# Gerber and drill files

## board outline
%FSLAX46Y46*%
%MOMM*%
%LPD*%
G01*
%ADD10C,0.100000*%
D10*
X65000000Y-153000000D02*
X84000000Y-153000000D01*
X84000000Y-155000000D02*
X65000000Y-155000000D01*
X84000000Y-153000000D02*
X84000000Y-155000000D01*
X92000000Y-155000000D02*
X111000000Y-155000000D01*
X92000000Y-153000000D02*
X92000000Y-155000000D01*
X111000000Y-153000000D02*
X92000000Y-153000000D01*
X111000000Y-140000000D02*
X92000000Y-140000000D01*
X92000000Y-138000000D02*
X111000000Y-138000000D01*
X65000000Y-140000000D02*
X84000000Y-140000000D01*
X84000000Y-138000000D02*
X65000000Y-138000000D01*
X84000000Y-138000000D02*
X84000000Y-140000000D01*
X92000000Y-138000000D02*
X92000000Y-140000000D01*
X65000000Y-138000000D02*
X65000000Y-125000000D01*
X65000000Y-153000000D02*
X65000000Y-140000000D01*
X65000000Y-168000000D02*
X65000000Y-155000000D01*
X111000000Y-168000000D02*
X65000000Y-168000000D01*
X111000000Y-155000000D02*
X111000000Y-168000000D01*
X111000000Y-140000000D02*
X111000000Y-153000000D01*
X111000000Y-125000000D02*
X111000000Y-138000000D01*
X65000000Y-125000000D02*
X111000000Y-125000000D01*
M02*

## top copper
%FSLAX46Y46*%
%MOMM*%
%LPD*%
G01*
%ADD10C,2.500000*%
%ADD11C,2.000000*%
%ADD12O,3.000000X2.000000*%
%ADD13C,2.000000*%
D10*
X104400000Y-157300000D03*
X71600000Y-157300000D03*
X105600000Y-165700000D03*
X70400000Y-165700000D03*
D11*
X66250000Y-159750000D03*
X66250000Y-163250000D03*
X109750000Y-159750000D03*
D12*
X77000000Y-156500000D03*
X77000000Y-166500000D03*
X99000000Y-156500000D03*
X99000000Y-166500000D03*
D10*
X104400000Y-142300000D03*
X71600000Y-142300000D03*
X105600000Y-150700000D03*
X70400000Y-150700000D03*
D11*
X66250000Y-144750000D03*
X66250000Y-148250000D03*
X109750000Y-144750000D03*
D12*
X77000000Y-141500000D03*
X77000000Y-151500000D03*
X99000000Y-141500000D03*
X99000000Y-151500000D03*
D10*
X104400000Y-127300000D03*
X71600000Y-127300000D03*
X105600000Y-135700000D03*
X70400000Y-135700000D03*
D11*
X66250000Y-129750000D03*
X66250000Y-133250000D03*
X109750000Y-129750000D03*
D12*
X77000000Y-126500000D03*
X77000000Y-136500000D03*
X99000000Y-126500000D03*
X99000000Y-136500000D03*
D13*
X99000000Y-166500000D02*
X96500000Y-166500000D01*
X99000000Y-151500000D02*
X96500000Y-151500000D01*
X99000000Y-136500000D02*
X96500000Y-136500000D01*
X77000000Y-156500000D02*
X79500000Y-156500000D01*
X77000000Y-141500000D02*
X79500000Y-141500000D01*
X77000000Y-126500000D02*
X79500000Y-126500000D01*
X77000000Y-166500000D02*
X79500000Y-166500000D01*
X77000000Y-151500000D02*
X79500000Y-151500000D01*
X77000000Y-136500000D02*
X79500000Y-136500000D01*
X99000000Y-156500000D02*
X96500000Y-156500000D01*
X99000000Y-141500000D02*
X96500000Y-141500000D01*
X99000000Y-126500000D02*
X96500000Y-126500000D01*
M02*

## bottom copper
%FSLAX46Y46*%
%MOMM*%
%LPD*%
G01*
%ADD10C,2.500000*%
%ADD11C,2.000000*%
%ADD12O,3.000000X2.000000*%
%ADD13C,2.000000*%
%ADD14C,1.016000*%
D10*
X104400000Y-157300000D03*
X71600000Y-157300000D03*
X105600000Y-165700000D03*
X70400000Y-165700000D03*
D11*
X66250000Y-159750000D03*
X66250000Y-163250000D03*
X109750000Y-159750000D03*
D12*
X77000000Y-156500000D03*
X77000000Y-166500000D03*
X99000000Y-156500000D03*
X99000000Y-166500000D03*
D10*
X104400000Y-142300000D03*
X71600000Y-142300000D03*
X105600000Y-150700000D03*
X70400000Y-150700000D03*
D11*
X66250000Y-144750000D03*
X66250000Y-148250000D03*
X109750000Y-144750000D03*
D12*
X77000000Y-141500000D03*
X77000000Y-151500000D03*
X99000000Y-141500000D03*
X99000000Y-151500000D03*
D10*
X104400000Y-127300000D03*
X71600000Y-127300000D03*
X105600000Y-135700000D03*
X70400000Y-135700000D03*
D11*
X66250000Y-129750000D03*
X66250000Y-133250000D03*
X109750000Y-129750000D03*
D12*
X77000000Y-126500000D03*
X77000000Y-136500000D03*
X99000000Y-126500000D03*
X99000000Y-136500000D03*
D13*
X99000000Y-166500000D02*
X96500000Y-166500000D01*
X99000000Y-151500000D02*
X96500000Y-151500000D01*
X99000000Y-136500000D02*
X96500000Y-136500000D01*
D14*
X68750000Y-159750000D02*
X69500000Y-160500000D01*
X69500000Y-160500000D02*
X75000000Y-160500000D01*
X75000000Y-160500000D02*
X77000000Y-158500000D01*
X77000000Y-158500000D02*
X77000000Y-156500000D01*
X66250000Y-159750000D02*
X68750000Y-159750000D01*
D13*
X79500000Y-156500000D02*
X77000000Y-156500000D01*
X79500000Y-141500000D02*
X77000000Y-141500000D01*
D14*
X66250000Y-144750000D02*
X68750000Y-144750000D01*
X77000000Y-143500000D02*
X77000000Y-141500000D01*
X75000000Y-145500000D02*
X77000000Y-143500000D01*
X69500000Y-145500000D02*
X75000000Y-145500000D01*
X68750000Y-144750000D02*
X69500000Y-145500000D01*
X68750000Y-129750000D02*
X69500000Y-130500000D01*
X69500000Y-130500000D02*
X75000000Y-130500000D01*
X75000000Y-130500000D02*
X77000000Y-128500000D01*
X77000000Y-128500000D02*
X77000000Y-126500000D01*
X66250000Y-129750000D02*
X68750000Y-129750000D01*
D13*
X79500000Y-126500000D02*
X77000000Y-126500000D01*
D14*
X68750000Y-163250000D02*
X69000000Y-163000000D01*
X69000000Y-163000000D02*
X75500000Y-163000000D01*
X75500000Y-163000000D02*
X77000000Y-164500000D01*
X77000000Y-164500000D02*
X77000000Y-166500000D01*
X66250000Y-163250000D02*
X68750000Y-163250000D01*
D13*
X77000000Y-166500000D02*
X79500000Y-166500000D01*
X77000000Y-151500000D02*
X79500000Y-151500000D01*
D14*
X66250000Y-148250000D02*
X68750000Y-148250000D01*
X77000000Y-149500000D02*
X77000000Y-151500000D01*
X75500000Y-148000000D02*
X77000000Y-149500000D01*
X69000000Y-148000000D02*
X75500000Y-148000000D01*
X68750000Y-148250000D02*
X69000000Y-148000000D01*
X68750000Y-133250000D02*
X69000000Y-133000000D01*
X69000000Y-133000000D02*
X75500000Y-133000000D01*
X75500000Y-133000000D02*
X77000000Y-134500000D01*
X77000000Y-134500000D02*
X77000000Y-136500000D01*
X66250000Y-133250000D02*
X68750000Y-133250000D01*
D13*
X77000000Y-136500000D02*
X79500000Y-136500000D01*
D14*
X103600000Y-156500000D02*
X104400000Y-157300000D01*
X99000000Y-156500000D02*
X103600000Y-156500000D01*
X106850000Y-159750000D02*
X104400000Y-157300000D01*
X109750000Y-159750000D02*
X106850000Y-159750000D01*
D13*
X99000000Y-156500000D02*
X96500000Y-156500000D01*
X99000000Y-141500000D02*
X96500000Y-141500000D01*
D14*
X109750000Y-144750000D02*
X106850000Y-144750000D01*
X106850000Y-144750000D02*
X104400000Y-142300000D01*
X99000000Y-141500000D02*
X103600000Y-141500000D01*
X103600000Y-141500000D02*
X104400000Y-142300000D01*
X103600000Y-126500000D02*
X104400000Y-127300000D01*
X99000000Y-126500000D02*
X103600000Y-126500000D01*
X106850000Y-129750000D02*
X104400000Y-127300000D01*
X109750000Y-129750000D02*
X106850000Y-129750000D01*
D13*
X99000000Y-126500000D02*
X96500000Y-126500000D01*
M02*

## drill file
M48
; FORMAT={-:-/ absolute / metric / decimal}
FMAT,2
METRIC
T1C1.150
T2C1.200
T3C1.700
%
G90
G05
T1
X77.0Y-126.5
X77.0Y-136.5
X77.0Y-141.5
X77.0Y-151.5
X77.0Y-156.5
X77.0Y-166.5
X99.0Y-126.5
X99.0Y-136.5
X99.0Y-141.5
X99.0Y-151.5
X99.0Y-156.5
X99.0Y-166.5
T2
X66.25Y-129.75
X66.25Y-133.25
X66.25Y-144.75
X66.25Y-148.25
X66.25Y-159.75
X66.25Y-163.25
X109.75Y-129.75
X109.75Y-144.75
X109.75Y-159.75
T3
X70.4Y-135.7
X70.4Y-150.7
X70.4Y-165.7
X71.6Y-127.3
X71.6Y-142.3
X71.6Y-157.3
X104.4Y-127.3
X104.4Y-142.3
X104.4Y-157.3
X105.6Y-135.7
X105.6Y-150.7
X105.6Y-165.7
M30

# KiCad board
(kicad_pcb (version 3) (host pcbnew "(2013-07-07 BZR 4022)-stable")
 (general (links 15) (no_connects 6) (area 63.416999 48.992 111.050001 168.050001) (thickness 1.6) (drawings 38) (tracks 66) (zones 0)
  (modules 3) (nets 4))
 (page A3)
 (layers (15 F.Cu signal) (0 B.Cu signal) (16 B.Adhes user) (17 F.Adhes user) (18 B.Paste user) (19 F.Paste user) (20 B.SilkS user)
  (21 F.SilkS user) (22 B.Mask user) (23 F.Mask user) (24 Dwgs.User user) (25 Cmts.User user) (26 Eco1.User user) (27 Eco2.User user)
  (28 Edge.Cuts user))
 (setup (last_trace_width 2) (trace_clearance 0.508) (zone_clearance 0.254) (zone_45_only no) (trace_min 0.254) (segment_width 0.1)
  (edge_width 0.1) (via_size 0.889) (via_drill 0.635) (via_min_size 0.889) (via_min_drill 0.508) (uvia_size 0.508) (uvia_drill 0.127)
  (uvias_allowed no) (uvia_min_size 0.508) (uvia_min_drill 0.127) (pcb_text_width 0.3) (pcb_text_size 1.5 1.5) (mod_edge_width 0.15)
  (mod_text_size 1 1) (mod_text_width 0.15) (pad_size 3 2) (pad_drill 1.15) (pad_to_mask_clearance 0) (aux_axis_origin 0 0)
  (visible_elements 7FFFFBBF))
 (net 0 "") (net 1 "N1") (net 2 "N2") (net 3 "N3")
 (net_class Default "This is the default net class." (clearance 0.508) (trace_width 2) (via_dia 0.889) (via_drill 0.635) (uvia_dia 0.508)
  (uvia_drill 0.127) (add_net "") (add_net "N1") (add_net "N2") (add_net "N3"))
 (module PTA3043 (layer F.Cu) (at 88 161.5)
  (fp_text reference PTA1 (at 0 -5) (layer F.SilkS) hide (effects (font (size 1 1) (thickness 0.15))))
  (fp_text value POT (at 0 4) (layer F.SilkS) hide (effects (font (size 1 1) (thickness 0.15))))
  (pad 7 thru_hole circle (at 16.4 -4.2) (size 2.5 2.5) (drill 1.7) (layers *.Cu *.Mask F.SilkS))
  (pad 6 thru_hole circle (at -16.4 -4.2) (size 2.5 2.5) (drill 1.7) (layers *.Cu *.Mask F.SilkS))
  (pad 5 thru_hole circle (at 17.6 4.2) (size 2.5 2.5) (drill 1.7) (layers *.Cu *.Mask F.SilkS))
  (pad 4 thru_hole circle (at -17.6 4.2) (size 2.5 2.5) (drill 1.7) (layers *.Cu *.Mask F.SilkS))
  (pad 1 thru_hole circle (at -21.75 -1.75) (size 2 2) (drill 1.2) (layers *.Cu *.Mask F.SilkS) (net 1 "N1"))
  (pad 2 thru_hole circle (at -21.75 1.75) (size 2 2) (drill 1.2) (layers *.Cu *.Mask F.SilkS) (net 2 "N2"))
  (pad 3 thru_hole circle (at 21.75 -1.75) (size 2 2) (drill 1.2) (layers *.Cu *.Mask F.SilkS) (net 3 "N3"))
  (pad 1 thru_hole oval (at -11 -5) (size 3 2) (drill 1.15) (layers *.Cu *.Mask F.SilkS) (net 1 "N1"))
  (pad 2 thru_hole oval (at -11 5) (size 3 2) (drill 1.15) (layers *.Cu *.Mask F.SilkS) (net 2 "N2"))
  (pad 3 thru_hole oval (at 11 -5) (size 3 2) (drill 1.15) (layers *.Cu *.Mask F.SilkS) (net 3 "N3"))
  (pad 8 thru_hole oval (at 11 5) (size 3 2) (drill 1.15) (layers *.Cu *.Mask F.SilkS)))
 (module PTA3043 (layer F.Cu) (at 88 146.5)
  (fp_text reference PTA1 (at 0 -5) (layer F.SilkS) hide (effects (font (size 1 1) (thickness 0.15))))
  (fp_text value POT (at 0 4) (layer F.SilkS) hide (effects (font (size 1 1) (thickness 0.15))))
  (pad 7 thru_hole circle (at 16.4 -4.2) (size 2.5 2.5) (drill 1.7) (layers *.Cu *.Mask F.SilkS))
  (pad 6 thru_hole circle (at -16.4 -4.2) (size 2.5 2.5) (drill 1.7) (layers *.Cu *.Mask F.SilkS))
  (pad 5 thru_hole circle (at 17.6 4.2) (size 2.5 2.5) (drill 1.7) (layers *.Cu *.Mask F.SilkS))
  (pad 4 thru_hole circle (at -17.6 4.2) (size 2.5 2.5) (drill 1.7) (layers *.Cu *.Mask F.SilkS))
  (pad 1 thru_hole circle (at -21.75 -1.75) (size 2 2) (drill 1.2) (layers *.Cu *.Mask F.SilkS) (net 1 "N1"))
  (pad 2 thru_hole circle (at -21.75 1.75) (size 2 2) (drill 1.2) (layers *.Cu *.Mask F.SilkS) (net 2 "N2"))
  (pad 3 thru_hole circle (at 21.75 -1.75) (size 2 2) (drill 1.2) (layers *.Cu *.Mask F.SilkS) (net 3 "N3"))
  (pad 1 thru_hole oval (at -11 -5) (size 3 2) (drill 1.15) (layers *.Cu *.Mask F.SilkS) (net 1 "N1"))
  (pad 2 thru_hole oval (at -11 5) (size 3 2) (drill 1.15) (layers *.Cu *.Mask F.SilkS) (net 2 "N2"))
  (pad 3 thru_hole oval (at 11 -5) (size 3 2) (drill 1.15) (layers *.Cu *.Mask F.SilkS) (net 3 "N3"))
  (pad 8 thru_hole oval (at 11 5) (size 3 2) (drill 1.15) (layers *.Cu *.Mask F.SilkS)))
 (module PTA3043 (layer F.Cu) (at 88 131.5)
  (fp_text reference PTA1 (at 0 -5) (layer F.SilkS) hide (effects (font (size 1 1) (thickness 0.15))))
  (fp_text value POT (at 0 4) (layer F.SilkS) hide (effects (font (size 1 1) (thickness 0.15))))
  (pad 7 thru_hole circle (at 16.4 -4.2) (size 2.5 2.5) (drill 1.7) (layers *.Cu *.Mask F.SilkS))
  (pad 6 thru_hole circle (at -16.4 -4.2) (size 2.5 2.5) (drill 1.7) (layers *.Cu *.Mask F.SilkS))
  (pad 5 thru_hole circle (at 17.6 4.2) (size 2.5 2.5) (drill 1.7) (layers *.Cu *.Mask F.SilkS))
  (pad 4 thru_hole circle (at -17.6 4.2) (size 2.5 2.5) (drill 1.7) (layers *.Cu *.Mask F.SilkS))
  (pad 1 thru_hole circle (at -21.75 -1.75) (size 2 2) (drill 1.2) (layers *.Cu *.Mask F.SilkS) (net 1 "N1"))
  (pad 2 thru_hole circle (at -21.75 1.75) (size 2 2) (drill 1.2) (layers *.Cu *.Mask F.SilkS) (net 2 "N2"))
  (pad 3 thru_hole circle (at 21.75 -1.75) (size 2 2) (drill 1.2) (layers *.Cu *.Mask F.SilkS) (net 3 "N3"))
  (pad 1 thru_hole oval (at -11 -5) (size 3 2) (drill 1.15) (layers *.Cu *.Mask F.SilkS) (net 1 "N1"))
  (pad 2 thru_hole oval (at -11 5) (size 3 2) (drill 1.15) (layers *.Cu *.Mask F.SilkS) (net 2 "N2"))
  (pad 3 thru_hole oval (at 11 -5) (size 3 2) (drill 1.15) (layers *.Cu *.Mask F.SilkS) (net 3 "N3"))
  (pad 8 thru_hole oval (at 11 5) (size 3 2) (drill 1.15) (layers *.Cu *.Mask F.SilkS)))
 (gr_line (start 65 153) (end 84 153) (angle 90) (layer Edge.Cuts) (width 0.1))
 (gr_line (start 84 155) (end 65 155) (angle 90) (layer Edge.Cuts) (width 0.1))
 (gr_line (start 84 153) (end 84 155) (angle 90) (layer Edge.Cuts) (width 0.1))
 (gr_line (start 92 155) (end 111 155) (angle 90) (layer Edge.Cuts) (width 0.1))
 (gr_line (start 92 153) (end 92 155) (angle 90) (layer Edge.Cuts) (width 0.1))
 (gr_line (start 111 153) (end 92 153) (angle 90) (layer Edge.Cuts) (width 0.1))
 (gr_line (start 111 140) (end 92 140) (angle 90) (layer Edge.Cuts) (width 0.1))
 (gr_line (start 92 138) (end 111 138) (angle 90) (layer Edge.Cuts) (width 0.1))
 (gr_line (start 65 140) (end 84 140) (angle 90) (layer Edge.Cuts) (width 0.1))
 (gr_line (start 84 138) (end 65 138) (angle 90) (layer Edge.Cuts) (width 0.1))
 (gr_line (start 84 138) (end 84 140) (angle 90) (layer Edge.Cuts) (width 0.1))
 (gr_line (start 92 138) (end 92 140) (angle 90) (layer Edge.Cuts) (width 0.1))
 (gr_line (start 65 138) (end 65 125) (angle 90) (layer Edge.Cuts) (width 0.1))
 (gr_line (start 65 153) (end 65 140) (angle 90) (layer Edge.Cuts) (width 0.1))
 (gr_line (start 65 168) (end 65 155) (angle 90) (layer Edge.Cuts) (width 0.1))
 (gr_line (start 111 168) (end 65 168) (angle 90) (layer Edge.Cuts) (width 0.1))
 (gr_line (start 111 155) (end 111 168) (angle 90) (layer Edge.Cuts) (width 0.1))
 (gr_line (start 111 140) (end 111 153) (angle 90) (layer Edge.Cuts) (width 0.1))
 (gr_line (start 111 125) (end 111 138) (angle 90) (layer Edge.Cuts) (width 0.1))
 (gr_line (start 65 125) (end 111 125) (angle 90) (layer Edge.Cuts) (width 0.1))
 (segment (start 99 166.5) (end 96.5 166.5) (width 2) (layer B.Cu) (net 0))
 (segment (start 99 166.5) (end 96.5 166.5) (width 2) (layer F.Cu) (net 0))
 (segment (start 99 151.5) (end 96.5 151.5) (width 2) (layer F.Cu) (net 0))
 (segment (start 99 151.5) (end 96.5 151.5) (width 2) (layer B.Cu) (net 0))
 (segment (start 99 136.5) (end 96.5 136.5) (width 2) (layer B.Cu) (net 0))
 (segment (start 99 136.5) (end 96.5 136.5) (width 2) (layer F.Cu) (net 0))
 (segment (start 68.75 159.75) (end 69.5 160.5) (width 1.016) (layer B.Cu) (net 1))
 (segment (start 69.5 160.5) (end 75 160.5) (width 1.016) (layer B.Cu) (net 1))
 (segment (start 75 160.5) (end 77 158.5) (width 1.016) (layer B.Cu) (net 1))
 (segment (start 77 158.5) (end 77 156.5) (width 1.016) (layer B.Cu) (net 1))
 (segment (start 66.25 159.75) (end 68.75 159.75) (width 1.016) (layer B.Cu) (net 1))
 (segment (start 79.5 156.5) (end 77 156.5) (width 2) (layer B.Cu) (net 1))
 (segment (start 77 156.5) (end 79.5 156.5) (width 2) (layer F.Cu) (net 1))
 (segment (start 77 141.5) (end 79.5 141.5) (width 2) (layer F.Cu) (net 1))
 (segment (start 79.5 141.5) (end 77 141.5) (width 2) (layer B.Cu) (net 1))
 (segment (start 66.25 144.75) (end 68.75 144.75) (width 1.016) (layer B.Cu) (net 1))
 (segment (start 77 143.5) (end 77 141.5) (width 1.016) (layer B.Cu) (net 1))
 (segment (start 75 145.5) (end 77 143.5) (width 1.016) (layer B.Cu) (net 1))
 (segment (start 69.5 145.5) (end 75 145.5) (width 1.016) (layer B.Cu) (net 1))
 (segment (start 68.75 144.75) (end 69.5 145.5) (width 1.016) (layer B.Cu) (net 1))
 (segment (start 68.75 129.75) (end 69.5 130.5) (width 1.016) (layer B.Cu) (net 1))
 (segment (start 69.5 130.5) (end 75 130.5) (width 1.016) (layer B.Cu) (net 1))
 (segment (start 75 130.5) (end 77 128.5) (width 1.016) (layer B.Cu) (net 1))
 (segment (start 77 128.5) (end 77 126.5) (width 1.016) (layer B.Cu) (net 1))
 (segment (start 66.25 129.75) (end 68.75 129.75) (width 1.016) (layer B.Cu) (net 1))
 (segment (start 79.5 126.5) (end 77 126.5) (width 2) (layer B.Cu) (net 1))
 (segment (start 77 126.5) (end 79.5 126.5) (width 2) (layer F.Cu) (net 1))
 (segment (start 68.75 163.25) (end 69 163) (width 1.016) (layer B.Cu) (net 2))
 (segment (start 69 163) (end 75.5 163) (width 1.016) (layer B.Cu) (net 2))
 (segment (start 75.5 163) (end 77 164.5) (width 1.016) (layer B.Cu) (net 2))
 (segment (start 77 164.5) (end 77 166.5) (width 1.016) (layer B.Cu) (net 2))
 (segment (start 66.25 163.25) (end 68.75 163.25) (width 1.016) (layer B.Cu) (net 2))
 (segment (start 77 166.5) (end 79.5 166.5) (width 2) (layer B.Cu) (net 2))
 (segment (start 77 166.5) (end 79.5 166.5) (width 2) (layer F.Cu) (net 2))
 (segment (start 77 151.5) (end 79.5 151.5) (width 2) (layer F.Cu) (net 2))
 (segment (start 77 151.5) (end 79.5 151.5) (width 2) (layer B.Cu) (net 2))
 (segment (start 66.25 148.25) (end 68.75 148.25) (width 1.016) (layer B.Cu) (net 2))
 (segment (start 77 149.5) (end 77 151.5) (width 1.016) (layer B.Cu) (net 2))
 (segment (start 75.5 148) (end 77 149.5) (width 1.016) (layer B.Cu) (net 2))
 (segment (start 69 148) (end 75.5 148) (width 1.016) (layer B.Cu) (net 2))
 (segment (start 68.75 148.25) (end 69 148) (width 1.016) (layer B.Cu) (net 2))
 (segment (start 68.75 133.25) (end 69 133) (width 1.016) (layer B.Cu) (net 2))
 (segment (start 69 133) (end 75.5 133) (width 1.016) (layer B.Cu) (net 2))
 (segment (start 75.5 133) (end 77 134.5) (width 1.016) (layer B.Cu) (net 2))
 (segment (start 77 134.5) (end 77 136.5) (width 1.016) (layer B.Cu) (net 2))
 (segment (start 66.25 133.25) (end 68.75 133.25) (width 1.016) (layer B.Cu) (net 2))
 (segment (start 77 136.5) (end 79.5 136.5) (width 2) (layer B.Cu) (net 2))
 (segment (start 77 136.5) (end 79.5 136.5) (width 2) (layer F.Cu) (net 2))
 (segment (start 103.6 156.5) (end 104.4 157.3) (width 1.016) (layer B.Cu) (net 3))
 (segment (start 99 156.5) (end 103.6 156.5) (width 1.016) (layer B.Cu) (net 3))
 (segment (start 106.85 159.75) (end 104.4 157.3) (width 1.016) (layer B.Cu) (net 3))
 (segment (start 109.75 159.75) (end 106.85 159.75) (width 1.016) (layer B.Cu) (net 3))
 (segment (start 99 156.5) (end 96.5 156.5) (width 2) (layer B.Cu) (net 3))
 (segment (start 99 156.5) (end 96.5 156.5) (width 2) (layer F.Cu) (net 3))
 (segment (start 99 141.5) (end 96.5 141.5) (width 2) (layer F.Cu) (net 3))
 (segment (start 99 141.5) (end 96.5 141.5) (width 2) (layer B.Cu) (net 3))
 (segment (start 109.75 144.75) (end 106.85 144.75) (width 1.016) (layer B.Cu) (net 3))
 (segment (start 106.85 144.75) (end 104.4 142.3) (width 1.016) (layer B.Cu) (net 3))
 (segment (start 99 141.5) (end 103.6 141.5) (width 1.016) (layer B.Cu) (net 3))
 (segment (start 103.6 141.5) (end 104.4 142.3) (width 1.016) (layer B.Cu) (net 3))
 (segment (start 103.6 126.5) (end 104.4 127.3) (width 1.016) (layer B.Cu) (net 3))
 (segment (start 99 126.5) (end 103.6 126.5) (width 1.016) (layer B.Cu) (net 3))
 (segment (start 106.85 129.75) (end 104.4 127.3) (width 1.016) (layer B.Cu) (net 3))
 (segment (start 109.75 129.75) (end 106.85 129.75) (width 1.016) (layer B.Cu) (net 3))
 (segment (start 99 126.5) (end 96.5 126.5) (width 2) (layer B.Cu) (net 3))
 (segment (start 99 126.5) (end 96.5 126.5) (width 2) (layer F.Cu) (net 3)))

